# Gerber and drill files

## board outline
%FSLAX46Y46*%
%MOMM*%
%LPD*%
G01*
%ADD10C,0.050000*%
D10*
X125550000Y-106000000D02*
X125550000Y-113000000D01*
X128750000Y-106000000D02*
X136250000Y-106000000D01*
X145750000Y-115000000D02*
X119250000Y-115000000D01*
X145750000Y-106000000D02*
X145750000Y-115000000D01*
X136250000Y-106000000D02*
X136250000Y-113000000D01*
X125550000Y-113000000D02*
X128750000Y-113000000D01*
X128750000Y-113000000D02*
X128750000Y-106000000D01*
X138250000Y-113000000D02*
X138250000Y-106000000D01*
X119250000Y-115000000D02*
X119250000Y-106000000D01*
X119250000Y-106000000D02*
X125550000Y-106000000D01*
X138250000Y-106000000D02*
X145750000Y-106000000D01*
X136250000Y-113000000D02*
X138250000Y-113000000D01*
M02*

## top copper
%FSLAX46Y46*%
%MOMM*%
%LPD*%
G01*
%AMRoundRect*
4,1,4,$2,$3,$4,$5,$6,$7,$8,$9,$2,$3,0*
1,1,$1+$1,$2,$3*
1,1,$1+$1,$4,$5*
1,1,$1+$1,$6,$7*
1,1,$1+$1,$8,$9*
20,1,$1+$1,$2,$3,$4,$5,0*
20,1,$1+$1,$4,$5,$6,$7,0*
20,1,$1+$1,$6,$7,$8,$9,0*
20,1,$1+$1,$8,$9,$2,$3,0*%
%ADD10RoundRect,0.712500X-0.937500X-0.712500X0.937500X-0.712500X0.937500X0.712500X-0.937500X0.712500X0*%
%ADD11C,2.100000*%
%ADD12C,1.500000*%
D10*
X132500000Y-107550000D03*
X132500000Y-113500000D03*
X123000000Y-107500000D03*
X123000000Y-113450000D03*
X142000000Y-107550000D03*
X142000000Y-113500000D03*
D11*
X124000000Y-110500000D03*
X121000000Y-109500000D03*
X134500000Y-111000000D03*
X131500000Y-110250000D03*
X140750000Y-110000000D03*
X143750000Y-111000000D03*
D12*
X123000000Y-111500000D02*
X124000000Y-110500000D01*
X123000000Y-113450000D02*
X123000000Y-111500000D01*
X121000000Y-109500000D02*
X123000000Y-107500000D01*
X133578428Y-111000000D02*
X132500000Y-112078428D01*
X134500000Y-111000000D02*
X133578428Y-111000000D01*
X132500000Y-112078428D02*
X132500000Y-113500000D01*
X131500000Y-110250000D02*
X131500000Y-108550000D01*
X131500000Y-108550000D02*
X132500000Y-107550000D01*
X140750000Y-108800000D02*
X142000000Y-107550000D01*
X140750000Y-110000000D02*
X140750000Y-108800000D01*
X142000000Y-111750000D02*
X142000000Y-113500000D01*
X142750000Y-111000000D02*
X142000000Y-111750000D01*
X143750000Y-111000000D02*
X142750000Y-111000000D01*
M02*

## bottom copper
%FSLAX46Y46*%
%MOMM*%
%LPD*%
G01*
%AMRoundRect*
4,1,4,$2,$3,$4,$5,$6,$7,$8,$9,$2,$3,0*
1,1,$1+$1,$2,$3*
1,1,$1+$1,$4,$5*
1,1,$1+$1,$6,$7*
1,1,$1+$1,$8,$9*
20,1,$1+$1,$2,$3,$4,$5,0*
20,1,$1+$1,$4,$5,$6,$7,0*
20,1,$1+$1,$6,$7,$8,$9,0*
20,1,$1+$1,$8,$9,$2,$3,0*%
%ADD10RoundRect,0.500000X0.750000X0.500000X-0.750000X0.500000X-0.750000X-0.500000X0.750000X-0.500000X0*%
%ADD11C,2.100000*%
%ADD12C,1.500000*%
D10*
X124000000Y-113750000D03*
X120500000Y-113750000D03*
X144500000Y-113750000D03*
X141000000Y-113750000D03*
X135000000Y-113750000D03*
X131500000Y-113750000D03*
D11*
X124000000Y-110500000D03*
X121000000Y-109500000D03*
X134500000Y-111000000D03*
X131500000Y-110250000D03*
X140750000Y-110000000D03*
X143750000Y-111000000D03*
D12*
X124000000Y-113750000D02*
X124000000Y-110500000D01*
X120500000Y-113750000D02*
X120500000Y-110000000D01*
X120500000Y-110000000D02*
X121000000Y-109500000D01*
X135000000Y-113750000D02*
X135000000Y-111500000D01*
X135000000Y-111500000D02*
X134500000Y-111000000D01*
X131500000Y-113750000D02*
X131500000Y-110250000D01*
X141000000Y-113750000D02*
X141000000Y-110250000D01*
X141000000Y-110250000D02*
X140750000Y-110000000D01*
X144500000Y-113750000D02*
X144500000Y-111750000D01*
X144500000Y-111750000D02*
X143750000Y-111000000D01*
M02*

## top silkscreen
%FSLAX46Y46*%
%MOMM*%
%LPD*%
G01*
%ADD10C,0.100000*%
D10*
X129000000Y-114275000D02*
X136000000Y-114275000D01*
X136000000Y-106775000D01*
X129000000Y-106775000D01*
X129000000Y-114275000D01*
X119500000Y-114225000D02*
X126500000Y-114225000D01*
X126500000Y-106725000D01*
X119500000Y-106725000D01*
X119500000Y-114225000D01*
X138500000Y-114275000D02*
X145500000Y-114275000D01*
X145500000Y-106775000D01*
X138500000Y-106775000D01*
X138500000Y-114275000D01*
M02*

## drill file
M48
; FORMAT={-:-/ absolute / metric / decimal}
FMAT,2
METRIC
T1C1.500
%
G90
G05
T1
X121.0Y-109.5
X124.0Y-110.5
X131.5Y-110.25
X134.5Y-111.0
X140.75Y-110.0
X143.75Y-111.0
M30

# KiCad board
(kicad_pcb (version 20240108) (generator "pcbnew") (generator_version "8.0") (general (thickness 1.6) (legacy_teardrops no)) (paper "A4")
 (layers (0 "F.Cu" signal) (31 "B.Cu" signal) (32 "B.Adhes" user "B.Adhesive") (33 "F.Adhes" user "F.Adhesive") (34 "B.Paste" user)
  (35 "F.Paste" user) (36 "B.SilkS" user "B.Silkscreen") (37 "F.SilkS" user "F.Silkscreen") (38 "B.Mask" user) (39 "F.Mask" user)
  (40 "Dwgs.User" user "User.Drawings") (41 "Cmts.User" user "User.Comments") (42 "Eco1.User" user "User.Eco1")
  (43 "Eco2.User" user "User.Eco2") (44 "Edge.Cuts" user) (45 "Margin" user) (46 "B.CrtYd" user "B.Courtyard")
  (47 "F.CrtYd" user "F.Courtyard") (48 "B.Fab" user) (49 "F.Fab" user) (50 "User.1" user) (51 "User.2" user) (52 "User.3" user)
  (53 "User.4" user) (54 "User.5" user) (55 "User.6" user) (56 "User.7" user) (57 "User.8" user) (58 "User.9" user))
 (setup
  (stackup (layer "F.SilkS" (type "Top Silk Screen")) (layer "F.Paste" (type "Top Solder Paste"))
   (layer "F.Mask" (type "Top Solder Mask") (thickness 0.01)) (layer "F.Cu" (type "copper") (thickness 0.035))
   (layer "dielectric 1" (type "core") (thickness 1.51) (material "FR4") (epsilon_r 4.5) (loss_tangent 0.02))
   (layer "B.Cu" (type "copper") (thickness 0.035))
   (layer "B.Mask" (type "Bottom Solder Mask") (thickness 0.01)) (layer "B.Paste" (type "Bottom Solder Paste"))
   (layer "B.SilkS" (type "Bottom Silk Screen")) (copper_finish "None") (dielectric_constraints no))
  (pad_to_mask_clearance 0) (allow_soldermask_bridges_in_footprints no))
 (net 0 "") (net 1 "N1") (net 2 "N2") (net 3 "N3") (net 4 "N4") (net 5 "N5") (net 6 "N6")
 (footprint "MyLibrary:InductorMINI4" (layer "F.Cu") (at 132.5 110.525)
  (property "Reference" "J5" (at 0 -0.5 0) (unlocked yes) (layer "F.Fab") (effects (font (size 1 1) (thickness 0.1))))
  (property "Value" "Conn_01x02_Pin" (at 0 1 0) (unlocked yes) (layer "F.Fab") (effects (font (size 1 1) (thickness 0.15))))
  (fp_rect (start -3.5 3.75) (end 3.5 -3.75) (stroke (width 0.1) (type default)) (fill none) (layer "F.SilkS"))
  (pad "1" smd roundrect (at 0 -2.975) (size 3.3 2.85) (layers "F.Cu" "F.Paste" "F.Mask") (roundrect_rratio 0.25) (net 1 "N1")
   (thermal_bridge_angle 45))
  (pad "2" smd roundrect (at 0 2.975) (size 3.3 2.85) (layers "F.Cu" "F.Paste" "F.Mask") (roundrect_rratio 0.25) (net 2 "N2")
   (thermal_bridge_angle 45)))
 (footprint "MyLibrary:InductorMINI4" (layer "F.Cu") (at 123 110.475)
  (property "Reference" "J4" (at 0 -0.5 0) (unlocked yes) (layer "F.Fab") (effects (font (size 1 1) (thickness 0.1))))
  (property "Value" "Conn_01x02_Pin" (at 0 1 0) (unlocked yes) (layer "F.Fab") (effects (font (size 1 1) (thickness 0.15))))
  (fp_rect (start -3.5 3.75) (end 3.5 -3.75) (stroke (width 0.1) (type default)) (fill none) (layer "F.SilkS"))
  (pad "1" smd roundrect (at 0 -2.975) (size 3.3 2.85) (layers "F.Cu" "F.Paste" "F.Mask") (roundrect_rratio 0.25) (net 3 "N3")
   (thermal_bridge_angle 45))
  (pad "2" smd roundrect (at 0 2.975) (size 3.3 2.85) (layers "F.Cu" "F.Paste" "F.Mask") (roundrect_rratio 0.25) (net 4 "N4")
   (thermal_bridge_angle 45)))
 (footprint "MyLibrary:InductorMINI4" (layer "F.Cu") (at 142 110.525)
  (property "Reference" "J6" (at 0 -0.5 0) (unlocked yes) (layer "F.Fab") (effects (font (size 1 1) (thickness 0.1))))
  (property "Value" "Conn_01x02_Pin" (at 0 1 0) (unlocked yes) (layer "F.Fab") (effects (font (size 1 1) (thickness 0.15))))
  (fp_rect (start -3.5 3.75) (end 3.5 -3.75) (stroke (width 0.1) (type default)) (fill none) (layer "F.SilkS"))
  (pad "1" smd roundrect (at 0 -2.975) (size 3.3 2.85) (layers "F.Cu" "F.Paste" "F.Mask") (roundrect_rratio 0.25) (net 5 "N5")
   (thermal_bridge_angle 45))
  (pad "2" smd roundrect (at 0 2.975) (size 3.3 2.85) (layers "F.Cu" "F.Paste" "F.Mask") (roundrect_rratio 0.25) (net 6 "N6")
   (thermal_bridge_angle 45)))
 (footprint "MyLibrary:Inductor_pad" (layer "B.Cu") (at 122.25 113.75 180)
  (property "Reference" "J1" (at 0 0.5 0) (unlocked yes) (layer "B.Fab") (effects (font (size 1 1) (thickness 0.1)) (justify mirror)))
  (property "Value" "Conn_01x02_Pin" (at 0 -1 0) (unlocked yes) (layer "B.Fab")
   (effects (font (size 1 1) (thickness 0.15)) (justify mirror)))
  (pad "1" smd roundrect (at -1.75 0 180) (size 2.5 2) (layers "B.Cu" "B.Paste" "B.Mask") (roundrect_rratio 0.25) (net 4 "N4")
   (thermal_bridge_angle 45))
  (pad "2" smd roundrect (at 1.75 0 180) (size 2.5 2) (layers "B.Cu" "B.Paste" "B.Mask") (roundrect_rratio 0.25) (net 3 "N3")
   (thermal_bridge_angle 45)))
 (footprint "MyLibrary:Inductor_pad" (layer "B.Cu") (at 142.75 113.75 180)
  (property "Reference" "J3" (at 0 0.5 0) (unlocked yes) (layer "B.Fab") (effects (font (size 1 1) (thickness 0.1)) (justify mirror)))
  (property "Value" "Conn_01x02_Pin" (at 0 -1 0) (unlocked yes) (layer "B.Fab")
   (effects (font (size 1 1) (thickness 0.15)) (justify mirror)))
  (pad "1" smd roundrect (at -1.75 0 180) (size 2.5 2) (layers "B.Cu" "B.Paste" "B.Mask") (roundrect_rratio 0.25) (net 6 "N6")
   (thermal_bridge_angle 45))
  (pad "2" smd roundrect (at 1.75 0 180) (size 2.5 2) (layers "B.Cu" "B.Paste" "B.Mask") (roundrect_rratio 0.25) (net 5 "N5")
   (thermal_bridge_angle 45)))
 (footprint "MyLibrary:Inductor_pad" (layer "B.Cu") (at 133.25 113.75 180)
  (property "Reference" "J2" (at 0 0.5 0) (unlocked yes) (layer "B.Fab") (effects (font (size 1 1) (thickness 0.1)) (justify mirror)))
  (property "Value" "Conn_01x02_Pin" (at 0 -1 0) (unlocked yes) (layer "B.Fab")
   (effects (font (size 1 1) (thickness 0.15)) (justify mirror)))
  (pad "1" smd roundrect (at -1.75 0 180) (size 2.5 2) (layers "B.Cu" "B.Paste" "B.Mask") (roundrect_rratio 0.25) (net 2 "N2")
   (thermal_bridge_angle 45))
  (pad "2" smd roundrect (at 1.75 0 180) (size 2.5 2) (layers "B.Cu" "B.Paste" "B.Mask") (roundrect_rratio 0.25) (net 1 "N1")
   (thermal_bridge_angle 45)))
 (gr_line (start 125.55 106) (end 125.55 113) (stroke (width 0.05) (type default)) (layer "Edge.Cuts"))
 (gr_line (start 128.75 106) (end 136.25 106) (stroke (width 0.05) (type default)) (layer "Edge.Cuts"))
 (gr_line (start 145.75 115) (end 119.25 115) (stroke (width 0.05) (type default)) (layer "Edge.Cuts"))
 (gr_line (start 145.75 106) (end 145.75 115) (stroke (width 0.05) (type default)) (layer "Edge.Cuts"))
 (gr_line (start 136.25 106) (end 136.25 113) (stroke (width 0.05) (type default)) (layer "Edge.Cuts"))
 (gr_line (start 125.55 113) (end 128.75 113) (stroke (width 0.05) (type default)) (layer "Edge.Cuts"))
 (gr_line (start 128.75 113) (end 128.75 106) (stroke (width 0.05) (type default)) (layer "Edge.Cuts"))
 (gr_line (start 138.25 113) (end 138.25 106) (stroke (width 0.05) (type default)) (layer "Edge.Cuts"))
 (gr_line (start 119.25 115) (end 119.25 106) (stroke (width 0.05) (type default)) (layer "Edge.Cuts"))
 (gr_line (start 119.25 106) (end 125.55 106) (stroke (width 0.05) (type default)) (layer "Edge.Cuts"))
 (gr_line (start 138.25 106) (end 145.75 106) (stroke (width 0.05) (type default)) (layer "Edge.Cuts"))
 (gr_line (start 136.25 113) (end 138.25 113) (stroke (width 0.05) (type default)) (layer "Edge.Cuts"))
 (segment (start 123 111.5) (end 124 110.5) (width 1.5) (layer "F.Cu") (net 4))
 (segment (start 123 113.45) (end 123 111.5) (width 1.5) (layer "F.Cu") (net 4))
 (via (at 124 110.5) (size 2.1) (drill 1.5) (layers "F.Cu" "B.Cu") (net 4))
 (segment (start 124 113.75) (end 124 110.5) (width 1.5) (layer "B.Cu") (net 4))
 (segment (start 121 109.5) (end 123 107.5) (width 1.5) (layer "F.Cu") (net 3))
 (via (at 121 109.5) (size 2.1) (drill 1.5) (layers "F.Cu" "B.Cu") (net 3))
 (segment (start 120.5 113.75) (end 120.5 110) (width 1.5) (layer "B.Cu") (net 3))
 (segment (start 120.5 110) (end 121 109.5) (width 1.5) (layer "B.Cu") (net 3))
 (segment (start 133.578428 111) (end 132.5 112.078428) (width 1.5) (layer "F.Cu") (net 2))
 (segment (start 134.5 111) (end 133.578428 111) (width 1.5) (layer "F.Cu") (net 2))
 (segment (start 132.5 112.078428) (end 132.5 113.5) (width 1.5) (layer "F.Cu") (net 2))
 (via (at 134.5 111) (size 2.1) (drill 1.5) (layers "F.Cu" "B.Cu") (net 2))
 (segment (start 135 113.75) (end 135 111.5) (width 1.5) (layer "B.Cu") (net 2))
 (segment (start 135 111.5) (end 134.5 111) (width 1.5) (layer "B.Cu") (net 2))
 (segment (start 131.5 110.25) (end 131.5 108.55) (width 1.5) (layer "F.Cu") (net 1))
 (segment (start 131.5 108.55) (end 132.5 107.55) (width 1.5) (layer "F.Cu") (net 1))
 (via (at 131.5 110.25) (size 2.1) (drill 1.5) (layers "F.Cu" "B.Cu") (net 1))
 (segment (start 131.5 113.75) (end 131.5 110.25) (width 1.5) (layer "B.Cu") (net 1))
 (segment (start 140.75 108.8) (end 142 107.55) (width 1.5) (layer "F.Cu") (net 5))
 (segment (start 140.75 110) (end 140.75 108.8) (width 1.5) (layer "F.Cu") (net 5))
 (via (at 140.75 110) (size 2.1) (drill 1.5) (layers "F.Cu" "B.Cu") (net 5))
 (segment (start 141 113.75) (end 141 110.25) (width 1.5) (layer "B.Cu") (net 5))
 (segment (start 141 110.25) (end 140.75 110) (width 1.5) (layer "B.Cu") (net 5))
 (segment (start 142 111.75) (end 142 113.5) (width 1.5) (layer "F.Cu") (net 6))
 (segment (start 142.75 111) (end 142 111.75) (width 1.5) (layer "F.Cu") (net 6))
 (segment (start 143.75 111) (end 142.75 111) (width 1.5) (layer "F.Cu") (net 6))
 (via (at 143.75 111) (size 2.1) (drill 1.5) (layers "F.Cu" "B.Cu") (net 6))
 (segment (start 144.5 113.75) (end 144.5 111.75) (width 1.5) (layer "B.Cu") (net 6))
 (segment (start 144.5 111.75) (end 143.75 111) (width 1.5) (layer "B.Cu") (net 6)))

